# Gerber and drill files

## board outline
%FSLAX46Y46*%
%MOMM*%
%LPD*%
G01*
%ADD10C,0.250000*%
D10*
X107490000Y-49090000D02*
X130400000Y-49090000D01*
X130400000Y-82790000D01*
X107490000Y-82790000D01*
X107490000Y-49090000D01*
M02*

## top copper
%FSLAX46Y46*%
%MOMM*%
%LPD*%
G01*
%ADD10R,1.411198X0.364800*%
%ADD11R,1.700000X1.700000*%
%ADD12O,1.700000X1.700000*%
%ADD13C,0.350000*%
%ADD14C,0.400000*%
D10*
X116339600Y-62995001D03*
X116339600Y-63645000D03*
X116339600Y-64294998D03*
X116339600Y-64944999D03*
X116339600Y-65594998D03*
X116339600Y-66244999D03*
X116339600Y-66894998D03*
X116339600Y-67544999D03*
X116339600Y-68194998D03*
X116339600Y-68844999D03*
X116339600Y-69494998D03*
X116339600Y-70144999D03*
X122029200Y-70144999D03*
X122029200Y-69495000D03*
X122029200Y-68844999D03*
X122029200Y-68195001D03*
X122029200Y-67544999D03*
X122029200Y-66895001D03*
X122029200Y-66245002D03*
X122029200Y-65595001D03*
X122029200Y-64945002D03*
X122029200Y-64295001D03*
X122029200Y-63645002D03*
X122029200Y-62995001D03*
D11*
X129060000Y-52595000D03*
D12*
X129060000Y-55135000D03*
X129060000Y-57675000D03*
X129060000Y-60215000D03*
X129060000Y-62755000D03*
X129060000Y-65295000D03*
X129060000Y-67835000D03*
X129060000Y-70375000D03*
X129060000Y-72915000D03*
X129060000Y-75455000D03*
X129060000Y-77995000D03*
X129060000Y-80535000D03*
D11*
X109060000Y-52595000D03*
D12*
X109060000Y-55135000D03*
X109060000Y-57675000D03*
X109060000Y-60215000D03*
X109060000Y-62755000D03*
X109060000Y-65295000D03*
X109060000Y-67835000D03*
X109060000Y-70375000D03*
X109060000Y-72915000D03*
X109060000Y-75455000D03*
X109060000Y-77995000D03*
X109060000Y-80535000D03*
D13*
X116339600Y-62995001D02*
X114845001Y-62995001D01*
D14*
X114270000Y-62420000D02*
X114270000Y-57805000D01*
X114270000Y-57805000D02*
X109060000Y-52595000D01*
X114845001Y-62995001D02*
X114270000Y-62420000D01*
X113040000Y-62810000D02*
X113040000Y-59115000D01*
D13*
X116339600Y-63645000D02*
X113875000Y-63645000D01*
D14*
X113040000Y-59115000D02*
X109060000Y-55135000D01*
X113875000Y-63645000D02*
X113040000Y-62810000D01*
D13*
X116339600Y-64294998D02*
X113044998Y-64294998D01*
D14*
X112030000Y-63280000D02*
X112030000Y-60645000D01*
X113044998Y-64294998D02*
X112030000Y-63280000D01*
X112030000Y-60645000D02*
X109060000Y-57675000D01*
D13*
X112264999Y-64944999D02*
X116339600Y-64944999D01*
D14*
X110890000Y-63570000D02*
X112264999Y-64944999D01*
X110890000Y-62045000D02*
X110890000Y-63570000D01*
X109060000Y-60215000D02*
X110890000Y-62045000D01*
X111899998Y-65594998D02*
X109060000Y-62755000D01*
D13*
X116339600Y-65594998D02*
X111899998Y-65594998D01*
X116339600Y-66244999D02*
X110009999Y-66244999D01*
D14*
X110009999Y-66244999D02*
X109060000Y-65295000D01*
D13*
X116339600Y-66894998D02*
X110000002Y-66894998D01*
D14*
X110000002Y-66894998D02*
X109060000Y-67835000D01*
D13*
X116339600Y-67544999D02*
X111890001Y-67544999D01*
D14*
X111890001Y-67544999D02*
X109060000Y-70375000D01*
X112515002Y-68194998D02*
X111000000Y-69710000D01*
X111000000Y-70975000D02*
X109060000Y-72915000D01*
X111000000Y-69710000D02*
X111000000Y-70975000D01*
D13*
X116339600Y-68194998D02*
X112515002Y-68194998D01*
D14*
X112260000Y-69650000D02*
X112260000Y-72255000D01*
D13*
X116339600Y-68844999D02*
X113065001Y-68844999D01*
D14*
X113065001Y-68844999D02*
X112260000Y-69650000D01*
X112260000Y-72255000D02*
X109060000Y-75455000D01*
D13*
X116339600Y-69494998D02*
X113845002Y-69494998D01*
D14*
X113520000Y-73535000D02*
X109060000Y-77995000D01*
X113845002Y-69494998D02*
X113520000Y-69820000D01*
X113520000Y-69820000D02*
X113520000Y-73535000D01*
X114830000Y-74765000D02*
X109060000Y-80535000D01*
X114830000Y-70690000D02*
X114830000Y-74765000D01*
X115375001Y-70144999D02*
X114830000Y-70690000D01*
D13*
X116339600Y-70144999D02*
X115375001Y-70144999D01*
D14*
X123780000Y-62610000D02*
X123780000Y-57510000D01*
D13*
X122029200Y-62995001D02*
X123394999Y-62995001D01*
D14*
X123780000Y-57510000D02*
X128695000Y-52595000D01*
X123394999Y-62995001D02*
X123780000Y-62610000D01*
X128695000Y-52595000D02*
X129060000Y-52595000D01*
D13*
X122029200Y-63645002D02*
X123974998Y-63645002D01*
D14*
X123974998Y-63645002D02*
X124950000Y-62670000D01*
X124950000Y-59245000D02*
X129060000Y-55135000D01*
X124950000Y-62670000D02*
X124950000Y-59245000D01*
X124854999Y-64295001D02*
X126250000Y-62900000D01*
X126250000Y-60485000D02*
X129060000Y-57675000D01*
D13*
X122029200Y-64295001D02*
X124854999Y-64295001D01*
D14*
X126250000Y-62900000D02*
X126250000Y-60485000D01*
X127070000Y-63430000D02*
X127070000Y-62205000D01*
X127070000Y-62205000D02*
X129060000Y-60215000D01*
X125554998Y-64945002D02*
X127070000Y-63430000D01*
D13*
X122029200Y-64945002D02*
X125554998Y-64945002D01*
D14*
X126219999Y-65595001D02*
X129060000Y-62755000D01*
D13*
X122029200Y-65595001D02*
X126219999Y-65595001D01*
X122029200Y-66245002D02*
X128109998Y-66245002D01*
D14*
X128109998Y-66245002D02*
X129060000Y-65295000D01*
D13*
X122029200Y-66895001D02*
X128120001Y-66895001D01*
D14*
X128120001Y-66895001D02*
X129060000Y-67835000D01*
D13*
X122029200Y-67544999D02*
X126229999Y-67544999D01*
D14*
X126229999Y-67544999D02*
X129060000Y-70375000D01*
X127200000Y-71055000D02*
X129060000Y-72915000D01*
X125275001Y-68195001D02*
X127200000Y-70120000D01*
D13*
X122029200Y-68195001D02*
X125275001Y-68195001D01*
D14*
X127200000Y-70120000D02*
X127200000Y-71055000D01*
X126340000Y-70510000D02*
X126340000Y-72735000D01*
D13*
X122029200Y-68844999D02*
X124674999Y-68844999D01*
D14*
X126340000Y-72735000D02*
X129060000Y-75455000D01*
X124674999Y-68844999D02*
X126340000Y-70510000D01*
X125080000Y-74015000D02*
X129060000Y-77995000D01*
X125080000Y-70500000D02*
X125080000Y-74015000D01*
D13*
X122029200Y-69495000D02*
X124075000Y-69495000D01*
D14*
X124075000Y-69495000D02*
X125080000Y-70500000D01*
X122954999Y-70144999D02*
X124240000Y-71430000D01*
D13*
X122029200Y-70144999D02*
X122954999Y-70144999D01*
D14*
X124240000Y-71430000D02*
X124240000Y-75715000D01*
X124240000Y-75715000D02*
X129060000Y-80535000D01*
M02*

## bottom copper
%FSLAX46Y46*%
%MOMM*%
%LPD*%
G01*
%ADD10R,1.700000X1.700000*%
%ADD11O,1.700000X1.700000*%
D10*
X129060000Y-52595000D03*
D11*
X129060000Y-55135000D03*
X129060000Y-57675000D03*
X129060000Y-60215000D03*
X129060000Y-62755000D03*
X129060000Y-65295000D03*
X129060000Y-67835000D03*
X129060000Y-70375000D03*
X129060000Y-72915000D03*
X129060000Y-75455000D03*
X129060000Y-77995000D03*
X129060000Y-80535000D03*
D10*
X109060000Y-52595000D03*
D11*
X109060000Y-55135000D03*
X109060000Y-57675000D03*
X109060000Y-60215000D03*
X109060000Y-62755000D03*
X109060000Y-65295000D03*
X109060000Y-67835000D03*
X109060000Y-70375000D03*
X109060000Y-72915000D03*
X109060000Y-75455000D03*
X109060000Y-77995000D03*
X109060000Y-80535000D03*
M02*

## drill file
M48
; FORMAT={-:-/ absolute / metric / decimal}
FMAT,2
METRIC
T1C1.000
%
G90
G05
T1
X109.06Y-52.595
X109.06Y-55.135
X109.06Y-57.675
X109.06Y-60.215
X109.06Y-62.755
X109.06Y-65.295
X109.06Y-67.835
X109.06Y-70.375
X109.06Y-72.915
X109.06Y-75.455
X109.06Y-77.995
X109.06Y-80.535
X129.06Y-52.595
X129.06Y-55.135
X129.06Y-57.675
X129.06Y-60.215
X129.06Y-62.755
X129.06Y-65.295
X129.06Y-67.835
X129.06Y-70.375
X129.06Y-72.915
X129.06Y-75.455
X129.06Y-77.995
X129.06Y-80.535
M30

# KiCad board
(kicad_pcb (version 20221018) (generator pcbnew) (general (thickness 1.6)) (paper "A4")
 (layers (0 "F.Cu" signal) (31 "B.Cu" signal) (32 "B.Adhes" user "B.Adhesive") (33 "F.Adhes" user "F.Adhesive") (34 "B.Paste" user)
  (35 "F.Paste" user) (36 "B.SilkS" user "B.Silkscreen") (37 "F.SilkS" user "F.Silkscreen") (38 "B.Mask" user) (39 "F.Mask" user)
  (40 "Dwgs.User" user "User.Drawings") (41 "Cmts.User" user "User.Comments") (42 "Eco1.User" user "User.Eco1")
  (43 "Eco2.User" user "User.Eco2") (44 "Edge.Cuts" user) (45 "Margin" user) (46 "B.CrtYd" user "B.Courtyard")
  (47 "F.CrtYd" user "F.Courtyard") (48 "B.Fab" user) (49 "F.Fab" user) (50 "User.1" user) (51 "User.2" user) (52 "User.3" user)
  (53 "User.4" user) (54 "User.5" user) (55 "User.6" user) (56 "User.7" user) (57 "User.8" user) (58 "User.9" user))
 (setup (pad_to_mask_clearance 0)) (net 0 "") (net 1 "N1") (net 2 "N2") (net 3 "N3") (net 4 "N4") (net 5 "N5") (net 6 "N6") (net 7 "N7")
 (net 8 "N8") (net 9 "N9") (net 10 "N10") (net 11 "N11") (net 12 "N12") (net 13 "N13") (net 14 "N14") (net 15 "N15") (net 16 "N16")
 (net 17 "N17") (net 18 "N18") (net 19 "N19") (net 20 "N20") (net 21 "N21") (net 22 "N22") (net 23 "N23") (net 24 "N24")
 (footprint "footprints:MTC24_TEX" (layer "F.Cu") (at 119.1844 66.57)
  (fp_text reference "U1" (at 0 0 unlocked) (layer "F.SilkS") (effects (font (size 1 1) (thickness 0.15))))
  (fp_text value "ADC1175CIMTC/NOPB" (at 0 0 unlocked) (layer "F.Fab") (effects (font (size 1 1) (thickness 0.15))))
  (pad "1" smd rect (at -2.8448 -3.574999) (size 1.411198 0.3648) (layers "F.Cu" "F.Paste" "F.Mask") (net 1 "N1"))
  (pad "2" smd rect (at -2.8448 -2.925) (size 1.411198 0.3648) (layers "F.Cu" "F.Paste" "F.Mask") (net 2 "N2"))
  (pad "3" smd rect (at -2.8448 -2.275002) (size 1.411198 0.3648) (layers "F.Cu" "F.Paste" "F.Mask") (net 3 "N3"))
  (pad "4" smd rect (at -2.8448 -1.625001) (size 1.411198 0.3648) (layers "F.Cu" "F.Paste" "F.Mask") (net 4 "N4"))
  (pad "5" smd rect (at -2.8448 -0.975002) (size 1.411198 0.3648) (layers "F.Cu" "F.Paste" "F.Mask") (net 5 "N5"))
  (pad "6" smd rect (at -2.8448 -0.325001) (size 1.411198 0.3648) (layers "F.Cu" "F.Paste" "F.Mask") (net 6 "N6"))
  (pad "7" smd rect (at -2.8448 0.324998) (size 1.411198 0.3648) (layers "F.Cu" "F.Paste" "F.Mask") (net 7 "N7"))
  (pad "8" smd rect (at -2.8448 0.974999) (size 1.411198 0.3648) (layers "F.Cu" "F.Paste" "F.Mask") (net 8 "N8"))
  (pad "9" smd rect (at -2.8448 1.624998) (size 1.411198 0.3648) (layers "F.Cu" "F.Paste" "F.Mask") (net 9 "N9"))
  (pad "10" smd rect (at -2.8448 2.274999) (size 1.411198 0.3648) (layers "F.Cu" "F.Paste" "F.Mask") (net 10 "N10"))
  (pad "11" smd rect (at -2.8448 2.924998) (size 1.411198 0.3648) (layers "F.Cu" "F.Paste" "F.Mask") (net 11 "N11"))
  (pad "12" smd rect (at -2.8448 3.574999) (size 1.411198 0.3648) (layers "F.Cu" "F.Paste" "F.Mask") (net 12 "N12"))
  (pad "13" smd rect (at 2.8448 3.574999) (size 1.411198 0.3648) (layers "F.Cu" "F.Paste" "F.Mask") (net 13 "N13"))
  (pad "14" smd rect (at 2.8448 2.925) (size 1.411198 0.3648) (layers "F.Cu" "F.Paste" "F.Mask") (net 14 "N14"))
  (pad "15" smd rect (at 2.8448 2.274999) (size 1.411198 0.3648) (layers "F.Cu" "F.Paste" "F.Mask") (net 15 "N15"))
  (pad "16" smd rect (at 2.8448 1.625001) (size 1.411198 0.3648) (layers "F.Cu" "F.Paste" "F.Mask") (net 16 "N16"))
  (pad "17" smd rect (at 2.8448 0.974999) (size 1.411198 0.3648) (layers "F.Cu" "F.Paste" "F.Mask") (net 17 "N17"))
  (pad "18" smd rect (at 2.8448 0.325001) (size 1.411198 0.3648) (layers "F.Cu" "F.Paste" "F.Mask") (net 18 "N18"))
  (pad "19" smd rect (at 2.8448 -0.324998) (size 1.411198 0.3648) (layers "F.Cu" "F.Paste" "F.Mask") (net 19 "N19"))
  (pad "20" smd rect (at 2.8448 -0.974999) (size 1.411198 0.3648) (layers "F.Cu" "F.Paste" "F.Mask") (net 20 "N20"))
  (pad "21" smd rect (at 2.8448 -1.624998) (size 1.411198 0.3648) (layers "F.Cu" "F.Paste" "F.Mask") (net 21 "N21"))
  (pad "22" smd rect (at 2.8448 -2.274999) (size 1.411198 0.3648) (layers "F.Cu" "F.Paste" "F.Mask") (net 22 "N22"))
  (pad "23" smd rect (at 2.8448 -2.924998) (size 1.411198 0.3648) (layers "F.Cu" "F.Paste" "F.Mask") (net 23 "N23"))
  (pad "24" smd rect (at 2.8448 -3.574999) (size 1.411198 0.3648) (layers "F.Cu" "F.Paste" "F.Mask") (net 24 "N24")))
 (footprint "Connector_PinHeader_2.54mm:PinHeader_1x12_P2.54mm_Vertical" (layer "F.Cu") (at 129.06 52.595)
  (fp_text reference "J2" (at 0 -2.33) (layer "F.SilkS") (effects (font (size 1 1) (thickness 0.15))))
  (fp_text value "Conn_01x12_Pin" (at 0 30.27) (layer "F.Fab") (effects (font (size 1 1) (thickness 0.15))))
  (pad "1" thru_hole rect (at 0 0) (size 1.7 1.7) (drill 1) (layers "*.Cu" "*.Mask") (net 24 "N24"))
  (pad "2" thru_hole oval (at 0 2.54) (size 1.7 1.7) (drill 1) (layers "*.Cu" "*.Mask") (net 23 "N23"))
  (pad "3" thru_hole oval (at 0 5.08) (size 1.7 1.7) (drill 1) (layers "*.Cu" "*.Mask") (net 22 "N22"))
  (pad "4" thru_hole oval (at 0 7.62) (size 1.7 1.7) (drill 1) (layers "*.Cu" "*.Mask") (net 21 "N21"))
  (pad "5" thru_hole oval (at 0 10.16) (size 1.7 1.7) (drill 1) (layers "*.Cu" "*.Mask") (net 20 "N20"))
  (pad "6" thru_hole oval (at 0 12.7) (size 1.7 1.7) (drill 1) (layers "*.Cu" "*.Mask") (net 19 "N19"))
  (pad "7" thru_hole oval (at 0 15.24) (size 1.7 1.7) (drill 1) (layers "*.Cu" "*.Mask") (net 18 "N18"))
  (pad "8" thru_hole oval (at 0 17.78) (size 1.7 1.7) (drill 1) (layers "*.Cu" "*.Mask") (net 17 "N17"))
  (pad "9" thru_hole oval (at 0 20.32) (size 1.7 1.7) (drill 1) (layers "*.Cu" "*.Mask") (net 16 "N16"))
  (pad "10" thru_hole oval (at 0 22.86) (size 1.7 1.7) (drill 1) (layers "*.Cu" "*.Mask") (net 15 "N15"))
  (pad "11" thru_hole oval (at 0 25.4) (size 1.7 1.7) (drill 1) (layers "*.Cu" "*.Mask") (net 14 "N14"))
  (pad "12" thru_hole oval (at 0 27.94) (size 1.7 1.7) (drill 1) (layers "*.Cu" "*.Mask") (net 13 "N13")))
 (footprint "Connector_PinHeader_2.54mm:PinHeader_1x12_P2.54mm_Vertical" (layer "F.Cu") (at 109.06 52.595)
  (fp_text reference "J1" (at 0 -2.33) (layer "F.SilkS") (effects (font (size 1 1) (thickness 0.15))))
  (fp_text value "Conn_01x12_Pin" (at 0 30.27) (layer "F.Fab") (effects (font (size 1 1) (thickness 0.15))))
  (pad "1" thru_hole rect (at 0 0) (size 1.7 1.7) (drill 1) (layers "*.Cu" "*.Mask") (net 1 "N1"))
  (pad "2" thru_hole oval (at 0 2.54) (size 1.7 1.7) (drill 1) (layers "*.Cu" "*.Mask") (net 2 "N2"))
  (pad "3" thru_hole oval (at 0 5.08) (size 1.7 1.7) (drill 1) (layers "*.Cu" "*.Mask") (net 3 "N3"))
  (pad "4" thru_hole oval (at 0 7.62) (size 1.7 1.7) (drill 1) (layers "*.Cu" "*.Mask") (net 4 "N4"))
  (pad "5" thru_hole oval (at 0 10.16) (size 1.7 1.7) (drill 1) (layers "*.Cu" "*.Mask") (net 5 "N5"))
  (pad "6" thru_hole oval (at 0 12.7) (size 1.7 1.7) (drill 1) (layers "*.Cu" "*.Mask") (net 6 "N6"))
  (pad "7" thru_hole oval (at 0 15.24) (size 1.7 1.7) (drill 1) (layers "*.Cu" "*.Mask") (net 7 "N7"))
  (pad "8" thru_hole oval (at 0 17.78) (size 1.7 1.7) (drill 1) (layers "*.Cu" "*.Mask") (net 8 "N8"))
  (pad "9" thru_hole oval (at 0 20.32) (size 1.7 1.7) (drill 1) (layers "*.Cu" "*.Mask") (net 9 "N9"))
  (pad "10" thru_hole oval (at 0 22.86) (size 1.7 1.7) (drill 1) (layers "*.Cu" "*.Mask") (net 10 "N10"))
  (pad "11" thru_hole oval (at 0 25.4) (size 1.7 1.7) (drill 1) (layers "*.Cu" "*.Mask") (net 11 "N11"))
  (pad "12" thru_hole oval (at 0 27.94) (size 1.7 1.7) (drill 1) (layers "*.Cu" "*.Mask") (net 12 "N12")))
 (gr_rect (start 107.49 49.09) (end 130.4 82.79) (stroke (width 0.25) (type default)) (fill none) (layer "Edge.Cuts"))
 (segment (start 116.3396 62.995001) (end 114.845001 62.995001) (width 0.35) (layer "F.Cu") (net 1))
 (segment (start 114.27 62.42) (end 114.27 57.805) (width 0.4) (layer "F.Cu") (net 1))
 (segment (start 114.27 57.805) (end 109.06 52.595) (width 0.4) (layer "F.Cu") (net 1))
 (segment (start 114.845001 62.995001) (end 114.27 62.42) (width 0.4) (layer "F.Cu") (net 1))
 (segment (start 113.04 62.81) (end 113.04 59.115) (width 0.4) (layer "F.Cu") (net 2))
 (segment (start 116.3396 63.645) (end 113.875 63.645) (width 0.35) (layer "F.Cu") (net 2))
 (segment (start 113.04 59.115) (end 109.06 55.135) (width 0.4) (layer "F.Cu") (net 2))
 (segment (start 113.875 63.645) (end 113.04 62.81) (width 0.4) (layer "F.Cu") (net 2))
 (segment (start 116.3396 64.294998) (end 113.044998 64.294998) (width 0.35) (layer "F.Cu") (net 3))
 (segment (start 112.03 63.28) (end 112.03 60.645) (width 0.4) (layer "F.Cu") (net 3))
 (segment (start 113.044998 64.294998) (end 112.03 63.28) (width 0.4) (layer "F.Cu") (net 3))
 (segment (start 112.03 60.645) (end 109.06 57.675) (width 0.4) (layer "F.Cu") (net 3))
 (segment (start 112.264999 64.944999) (end 116.3396 64.944999) (width 0.35) (layer "F.Cu") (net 4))
 (segment (start 110.89 63.57) (end 112.264999 64.944999) (width 0.4) (layer "F.Cu") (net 4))
 (segment (start 110.89 62.045) (end 110.89 63.57) (width 0.4) (layer "F.Cu") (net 4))
 (segment (start 109.06 60.215) (end 110.89 62.045) (width 0.4) (layer "F.Cu") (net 4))
 (segment (start 111.899998 65.594998) (end 109.06 62.755) (width 0.4) (layer "F.Cu") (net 5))
 (segment (start 116.3396 65.594998) (end 111.899998 65.594998) (width 0.35) (layer "F.Cu") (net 5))
 (segment (start 116.3396 66.244999) (end 110.009999 66.244999) (width 0.35) (layer "F.Cu") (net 6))
 (segment (start 110.009999 66.244999) (end 109.06 65.295) (width 0.4) (layer "F.Cu") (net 6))
 (segment (start 116.3396 66.894998) (end 110.000002 66.894998) (width 0.35) (layer "F.Cu") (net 7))
 (segment (start 110.000002 66.894998) (end 109.06 67.835) (width 0.4) (layer "F.Cu") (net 7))
 (segment (start 116.3396 67.544999) (end 111.890001 67.544999) (width 0.35) (layer "F.Cu") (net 8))
 (segment (start 111.890001 67.544999) (end 109.06 70.375) (width 0.4) (layer "F.Cu") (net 8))
 (segment (start 112.515002 68.194998) (end 111 69.71) (width 0.4) (layer "F.Cu") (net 9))
 (segment (start 111 70.975) (end 109.06 72.915) (width 0.4) (layer "F.Cu") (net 9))
 (segment (start 111 69.71) (end 111 70.975) (width 0.4) (layer "F.Cu") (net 9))
 (segment (start 116.3396 68.194998) (end 112.515002 68.194998) (width 0.35) (layer "F.Cu") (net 9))
 (segment (start 112.26 69.65) (end 112.26 72.255) (width 0.4) (layer "F.Cu") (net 10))
 (segment (start 116.3396 68.844999) (end 113.065001 68.844999) (width 0.35) (layer "F.Cu") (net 10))
 (segment (start 113.065001 68.844999) (end 112.26 69.65) (width 0.4) (layer "F.Cu") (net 10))
 (segment (start 112.26 72.255) (end 109.06 75.455) (width 0.4) (layer "F.Cu") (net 10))
 (segment (start 116.3396 69.494998) (end 113.845002 69.494998) (width 0.35) (layer "F.Cu") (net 11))
 (segment (start 113.52 73.535) (end 109.06 77.995) (width 0.4) (layer "F.Cu") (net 11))
 (segment (start 113.845002 69.494998) (end 113.52 69.82) (width 0.4) (layer "F.Cu") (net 11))
 (segment (start 113.52 69.82) (end 113.52 73.535) (width 0.4) (layer "F.Cu") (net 11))
 (segment (start 114.83 74.765) (end 109.06 80.535) (width 0.4) (layer "F.Cu") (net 12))
 (segment (start 114.83 70.69) (end 114.83 74.765) (width 0.4) (layer "F.Cu") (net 12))
 (segment (start 115.375001 70.144999) (end 114.83 70.69) (width 0.4) (layer "F.Cu") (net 12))
 (segment (start 116.3396 70.144999) (end 115.375001 70.144999) (width 0.35) (layer "F.Cu") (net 12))
 (segment (start 123.78 62.61) (end 123.78 57.51) (width 0.4) (layer "F.Cu") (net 24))
 (segment (start 122.0292 62.995001) (end 123.394999 62.995001) (width 0.35) (layer "F.Cu") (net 24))
 (segment (start 123.78 57.51) (end 128.695 52.595) (width 0.4) (layer "F.Cu") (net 24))
 (segment (start 123.394999 62.995001) (end 123.78 62.61) (width 0.4) (layer "F.Cu") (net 24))
 (segment (start 128.695 52.595) (end 129.06 52.595) (width 0.4) (layer "F.Cu") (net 24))
 (segment (start 122.0292 63.645002) (end 123.974998 63.645002) (width 0.35) (layer "F.Cu") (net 23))
 (segment (start 123.974998 63.645002) (end 124.95 62.67) (width 0.4) (layer "F.Cu") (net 23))
 (segment (start 124.95 59.245) (end 129.06 55.135) (width 0.4) (layer "F.Cu") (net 23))
 (segment (start 124.95 62.67) (end 124.95 59.245) (width 0.4) (layer "F.Cu") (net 23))
 (segment (start 124.854999 64.295001) (end 126.25 62.9) (width 0.4) (layer "F.Cu") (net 22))
 (segment (start 126.25 60.485) (end 129.06 57.675) (width 0.4) (layer "F.Cu") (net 22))
 (segment (start 122.0292 64.295001) (end 124.854999 64.295001) (width 0.35) (layer "F.Cu") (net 22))
 (segment (start 126.25 62.9) (end 126.25 60.485) (width 0.4) (layer "F.Cu") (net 22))
 (segment (start 127.07 63.43) (end 127.07 62.205) (width 0.4) (layer "F.Cu") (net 21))
 (segment (start 127.07 62.205) (end 129.06 60.215) (width 0.4) (layer "F.Cu") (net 21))
 (segment (start 125.554998 64.945002) (end 127.07 63.43) (width 0.4) (layer "F.Cu") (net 21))
 (segment (start 122.0292 64.945002) (end 125.554998 64.945002) (width 0.35) (layer "F.Cu") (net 21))
 (segment (start 126.219999 65.595001) (end 129.06 62.755) (width 0.4) (layer "F.Cu") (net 20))
 (segment (start 122.0292 65.595001) (end 126.219999 65.595001) (width 0.35) (layer "F.Cu") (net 20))
 (segment (start 122.0292 66.245002) (end 128.109998 66.245002) (width 0.35) (layer "F.Cu") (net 19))
 (segment (start 128.109998 66.245002) (end 129.06 65.295) (width 0.4) (layer "F.Cu") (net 19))
 (segment (start 122.0292 66.895001) (end 128.120001 66.895001) (width 0.35) (layer "F.Cu") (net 18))
 (segment (start 128.120001 66.895001) (end 129.06 67.835) (width 0.4) (layer "F.Cu") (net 18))
 (segment (start 122.0292 67.544999) (end 126.229999 67.544999) (width 0.35) (layer "F.Cu") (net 17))
 (segment (start 126.229999 67.544999) (end 129.06 70.375) (width 0.4) (layer "F.Cu") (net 17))
 (segment (start 127.2 71.055) (end 129.06 72.915) (width 0.4) (layer "F.Cu") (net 16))
 (segment (start 125.275001 68.195001) (end 127.2 70.12) (width 0.4) (layer "F.Cu") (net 16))
 (segment (start 122.0292 68.195001) (end 125.275001 68.195001) (width 0.35) (layer "F.Cu") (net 16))
 (segment (start 127.2 70.12) (end 127.2 71.055) (width 0.4) (layer "F.Cu") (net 16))
 (segment (start 126.34 70.51) (end 126.34 72.735) (width 0.4) (layer "F.Cu") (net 15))
 (segment (start 122.0292 68.844999) (end 124.674999 68.844999) (width 0.35) (layer "F.Cu") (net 15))
 (segment (start 126.34 72.735) (end 129.06 75.455) (width 0.4) (layer "F.Cu") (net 15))
 (segment (start 124.674999 68.844999) (end 126.34 70.51) (width 0.4) (layer "F.Cu") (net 15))
 (segment (start 125.08 74.015) (end 129.06 77.995) (width 0.4) (layer "F.Cu") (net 14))
 (segment (start 125.08 70.5) (end 125.08 74.015) (width 0.4) (layer "F.Cu") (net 14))
 (segment (start 122.0292 69.495) (end 124.075 69.495) (width 0.35) (layer "F.Cu") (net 14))
 (segment (start 124.075 69.495) (end 125.08 70.5) (width 0.4) (layer "F.Cu") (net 14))
 (segment (start 122.954999 70.144999) (end 124.24 71.43) (width 0.4) (layer "F.Cu") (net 13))
 (segment (start 122.0292 70.144999) (end 122.954999 70.144999) (width 0.35) (layer "F.Cu") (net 13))
 (segment (start 124.24 71.43) (end 124.24 75.715) (width 0.4) (layer "F.Cu") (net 13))
 (segment (start 124.24 75.715) (end 129.06 80.535) (width 0.4) (layer "F.Cu") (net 13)))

